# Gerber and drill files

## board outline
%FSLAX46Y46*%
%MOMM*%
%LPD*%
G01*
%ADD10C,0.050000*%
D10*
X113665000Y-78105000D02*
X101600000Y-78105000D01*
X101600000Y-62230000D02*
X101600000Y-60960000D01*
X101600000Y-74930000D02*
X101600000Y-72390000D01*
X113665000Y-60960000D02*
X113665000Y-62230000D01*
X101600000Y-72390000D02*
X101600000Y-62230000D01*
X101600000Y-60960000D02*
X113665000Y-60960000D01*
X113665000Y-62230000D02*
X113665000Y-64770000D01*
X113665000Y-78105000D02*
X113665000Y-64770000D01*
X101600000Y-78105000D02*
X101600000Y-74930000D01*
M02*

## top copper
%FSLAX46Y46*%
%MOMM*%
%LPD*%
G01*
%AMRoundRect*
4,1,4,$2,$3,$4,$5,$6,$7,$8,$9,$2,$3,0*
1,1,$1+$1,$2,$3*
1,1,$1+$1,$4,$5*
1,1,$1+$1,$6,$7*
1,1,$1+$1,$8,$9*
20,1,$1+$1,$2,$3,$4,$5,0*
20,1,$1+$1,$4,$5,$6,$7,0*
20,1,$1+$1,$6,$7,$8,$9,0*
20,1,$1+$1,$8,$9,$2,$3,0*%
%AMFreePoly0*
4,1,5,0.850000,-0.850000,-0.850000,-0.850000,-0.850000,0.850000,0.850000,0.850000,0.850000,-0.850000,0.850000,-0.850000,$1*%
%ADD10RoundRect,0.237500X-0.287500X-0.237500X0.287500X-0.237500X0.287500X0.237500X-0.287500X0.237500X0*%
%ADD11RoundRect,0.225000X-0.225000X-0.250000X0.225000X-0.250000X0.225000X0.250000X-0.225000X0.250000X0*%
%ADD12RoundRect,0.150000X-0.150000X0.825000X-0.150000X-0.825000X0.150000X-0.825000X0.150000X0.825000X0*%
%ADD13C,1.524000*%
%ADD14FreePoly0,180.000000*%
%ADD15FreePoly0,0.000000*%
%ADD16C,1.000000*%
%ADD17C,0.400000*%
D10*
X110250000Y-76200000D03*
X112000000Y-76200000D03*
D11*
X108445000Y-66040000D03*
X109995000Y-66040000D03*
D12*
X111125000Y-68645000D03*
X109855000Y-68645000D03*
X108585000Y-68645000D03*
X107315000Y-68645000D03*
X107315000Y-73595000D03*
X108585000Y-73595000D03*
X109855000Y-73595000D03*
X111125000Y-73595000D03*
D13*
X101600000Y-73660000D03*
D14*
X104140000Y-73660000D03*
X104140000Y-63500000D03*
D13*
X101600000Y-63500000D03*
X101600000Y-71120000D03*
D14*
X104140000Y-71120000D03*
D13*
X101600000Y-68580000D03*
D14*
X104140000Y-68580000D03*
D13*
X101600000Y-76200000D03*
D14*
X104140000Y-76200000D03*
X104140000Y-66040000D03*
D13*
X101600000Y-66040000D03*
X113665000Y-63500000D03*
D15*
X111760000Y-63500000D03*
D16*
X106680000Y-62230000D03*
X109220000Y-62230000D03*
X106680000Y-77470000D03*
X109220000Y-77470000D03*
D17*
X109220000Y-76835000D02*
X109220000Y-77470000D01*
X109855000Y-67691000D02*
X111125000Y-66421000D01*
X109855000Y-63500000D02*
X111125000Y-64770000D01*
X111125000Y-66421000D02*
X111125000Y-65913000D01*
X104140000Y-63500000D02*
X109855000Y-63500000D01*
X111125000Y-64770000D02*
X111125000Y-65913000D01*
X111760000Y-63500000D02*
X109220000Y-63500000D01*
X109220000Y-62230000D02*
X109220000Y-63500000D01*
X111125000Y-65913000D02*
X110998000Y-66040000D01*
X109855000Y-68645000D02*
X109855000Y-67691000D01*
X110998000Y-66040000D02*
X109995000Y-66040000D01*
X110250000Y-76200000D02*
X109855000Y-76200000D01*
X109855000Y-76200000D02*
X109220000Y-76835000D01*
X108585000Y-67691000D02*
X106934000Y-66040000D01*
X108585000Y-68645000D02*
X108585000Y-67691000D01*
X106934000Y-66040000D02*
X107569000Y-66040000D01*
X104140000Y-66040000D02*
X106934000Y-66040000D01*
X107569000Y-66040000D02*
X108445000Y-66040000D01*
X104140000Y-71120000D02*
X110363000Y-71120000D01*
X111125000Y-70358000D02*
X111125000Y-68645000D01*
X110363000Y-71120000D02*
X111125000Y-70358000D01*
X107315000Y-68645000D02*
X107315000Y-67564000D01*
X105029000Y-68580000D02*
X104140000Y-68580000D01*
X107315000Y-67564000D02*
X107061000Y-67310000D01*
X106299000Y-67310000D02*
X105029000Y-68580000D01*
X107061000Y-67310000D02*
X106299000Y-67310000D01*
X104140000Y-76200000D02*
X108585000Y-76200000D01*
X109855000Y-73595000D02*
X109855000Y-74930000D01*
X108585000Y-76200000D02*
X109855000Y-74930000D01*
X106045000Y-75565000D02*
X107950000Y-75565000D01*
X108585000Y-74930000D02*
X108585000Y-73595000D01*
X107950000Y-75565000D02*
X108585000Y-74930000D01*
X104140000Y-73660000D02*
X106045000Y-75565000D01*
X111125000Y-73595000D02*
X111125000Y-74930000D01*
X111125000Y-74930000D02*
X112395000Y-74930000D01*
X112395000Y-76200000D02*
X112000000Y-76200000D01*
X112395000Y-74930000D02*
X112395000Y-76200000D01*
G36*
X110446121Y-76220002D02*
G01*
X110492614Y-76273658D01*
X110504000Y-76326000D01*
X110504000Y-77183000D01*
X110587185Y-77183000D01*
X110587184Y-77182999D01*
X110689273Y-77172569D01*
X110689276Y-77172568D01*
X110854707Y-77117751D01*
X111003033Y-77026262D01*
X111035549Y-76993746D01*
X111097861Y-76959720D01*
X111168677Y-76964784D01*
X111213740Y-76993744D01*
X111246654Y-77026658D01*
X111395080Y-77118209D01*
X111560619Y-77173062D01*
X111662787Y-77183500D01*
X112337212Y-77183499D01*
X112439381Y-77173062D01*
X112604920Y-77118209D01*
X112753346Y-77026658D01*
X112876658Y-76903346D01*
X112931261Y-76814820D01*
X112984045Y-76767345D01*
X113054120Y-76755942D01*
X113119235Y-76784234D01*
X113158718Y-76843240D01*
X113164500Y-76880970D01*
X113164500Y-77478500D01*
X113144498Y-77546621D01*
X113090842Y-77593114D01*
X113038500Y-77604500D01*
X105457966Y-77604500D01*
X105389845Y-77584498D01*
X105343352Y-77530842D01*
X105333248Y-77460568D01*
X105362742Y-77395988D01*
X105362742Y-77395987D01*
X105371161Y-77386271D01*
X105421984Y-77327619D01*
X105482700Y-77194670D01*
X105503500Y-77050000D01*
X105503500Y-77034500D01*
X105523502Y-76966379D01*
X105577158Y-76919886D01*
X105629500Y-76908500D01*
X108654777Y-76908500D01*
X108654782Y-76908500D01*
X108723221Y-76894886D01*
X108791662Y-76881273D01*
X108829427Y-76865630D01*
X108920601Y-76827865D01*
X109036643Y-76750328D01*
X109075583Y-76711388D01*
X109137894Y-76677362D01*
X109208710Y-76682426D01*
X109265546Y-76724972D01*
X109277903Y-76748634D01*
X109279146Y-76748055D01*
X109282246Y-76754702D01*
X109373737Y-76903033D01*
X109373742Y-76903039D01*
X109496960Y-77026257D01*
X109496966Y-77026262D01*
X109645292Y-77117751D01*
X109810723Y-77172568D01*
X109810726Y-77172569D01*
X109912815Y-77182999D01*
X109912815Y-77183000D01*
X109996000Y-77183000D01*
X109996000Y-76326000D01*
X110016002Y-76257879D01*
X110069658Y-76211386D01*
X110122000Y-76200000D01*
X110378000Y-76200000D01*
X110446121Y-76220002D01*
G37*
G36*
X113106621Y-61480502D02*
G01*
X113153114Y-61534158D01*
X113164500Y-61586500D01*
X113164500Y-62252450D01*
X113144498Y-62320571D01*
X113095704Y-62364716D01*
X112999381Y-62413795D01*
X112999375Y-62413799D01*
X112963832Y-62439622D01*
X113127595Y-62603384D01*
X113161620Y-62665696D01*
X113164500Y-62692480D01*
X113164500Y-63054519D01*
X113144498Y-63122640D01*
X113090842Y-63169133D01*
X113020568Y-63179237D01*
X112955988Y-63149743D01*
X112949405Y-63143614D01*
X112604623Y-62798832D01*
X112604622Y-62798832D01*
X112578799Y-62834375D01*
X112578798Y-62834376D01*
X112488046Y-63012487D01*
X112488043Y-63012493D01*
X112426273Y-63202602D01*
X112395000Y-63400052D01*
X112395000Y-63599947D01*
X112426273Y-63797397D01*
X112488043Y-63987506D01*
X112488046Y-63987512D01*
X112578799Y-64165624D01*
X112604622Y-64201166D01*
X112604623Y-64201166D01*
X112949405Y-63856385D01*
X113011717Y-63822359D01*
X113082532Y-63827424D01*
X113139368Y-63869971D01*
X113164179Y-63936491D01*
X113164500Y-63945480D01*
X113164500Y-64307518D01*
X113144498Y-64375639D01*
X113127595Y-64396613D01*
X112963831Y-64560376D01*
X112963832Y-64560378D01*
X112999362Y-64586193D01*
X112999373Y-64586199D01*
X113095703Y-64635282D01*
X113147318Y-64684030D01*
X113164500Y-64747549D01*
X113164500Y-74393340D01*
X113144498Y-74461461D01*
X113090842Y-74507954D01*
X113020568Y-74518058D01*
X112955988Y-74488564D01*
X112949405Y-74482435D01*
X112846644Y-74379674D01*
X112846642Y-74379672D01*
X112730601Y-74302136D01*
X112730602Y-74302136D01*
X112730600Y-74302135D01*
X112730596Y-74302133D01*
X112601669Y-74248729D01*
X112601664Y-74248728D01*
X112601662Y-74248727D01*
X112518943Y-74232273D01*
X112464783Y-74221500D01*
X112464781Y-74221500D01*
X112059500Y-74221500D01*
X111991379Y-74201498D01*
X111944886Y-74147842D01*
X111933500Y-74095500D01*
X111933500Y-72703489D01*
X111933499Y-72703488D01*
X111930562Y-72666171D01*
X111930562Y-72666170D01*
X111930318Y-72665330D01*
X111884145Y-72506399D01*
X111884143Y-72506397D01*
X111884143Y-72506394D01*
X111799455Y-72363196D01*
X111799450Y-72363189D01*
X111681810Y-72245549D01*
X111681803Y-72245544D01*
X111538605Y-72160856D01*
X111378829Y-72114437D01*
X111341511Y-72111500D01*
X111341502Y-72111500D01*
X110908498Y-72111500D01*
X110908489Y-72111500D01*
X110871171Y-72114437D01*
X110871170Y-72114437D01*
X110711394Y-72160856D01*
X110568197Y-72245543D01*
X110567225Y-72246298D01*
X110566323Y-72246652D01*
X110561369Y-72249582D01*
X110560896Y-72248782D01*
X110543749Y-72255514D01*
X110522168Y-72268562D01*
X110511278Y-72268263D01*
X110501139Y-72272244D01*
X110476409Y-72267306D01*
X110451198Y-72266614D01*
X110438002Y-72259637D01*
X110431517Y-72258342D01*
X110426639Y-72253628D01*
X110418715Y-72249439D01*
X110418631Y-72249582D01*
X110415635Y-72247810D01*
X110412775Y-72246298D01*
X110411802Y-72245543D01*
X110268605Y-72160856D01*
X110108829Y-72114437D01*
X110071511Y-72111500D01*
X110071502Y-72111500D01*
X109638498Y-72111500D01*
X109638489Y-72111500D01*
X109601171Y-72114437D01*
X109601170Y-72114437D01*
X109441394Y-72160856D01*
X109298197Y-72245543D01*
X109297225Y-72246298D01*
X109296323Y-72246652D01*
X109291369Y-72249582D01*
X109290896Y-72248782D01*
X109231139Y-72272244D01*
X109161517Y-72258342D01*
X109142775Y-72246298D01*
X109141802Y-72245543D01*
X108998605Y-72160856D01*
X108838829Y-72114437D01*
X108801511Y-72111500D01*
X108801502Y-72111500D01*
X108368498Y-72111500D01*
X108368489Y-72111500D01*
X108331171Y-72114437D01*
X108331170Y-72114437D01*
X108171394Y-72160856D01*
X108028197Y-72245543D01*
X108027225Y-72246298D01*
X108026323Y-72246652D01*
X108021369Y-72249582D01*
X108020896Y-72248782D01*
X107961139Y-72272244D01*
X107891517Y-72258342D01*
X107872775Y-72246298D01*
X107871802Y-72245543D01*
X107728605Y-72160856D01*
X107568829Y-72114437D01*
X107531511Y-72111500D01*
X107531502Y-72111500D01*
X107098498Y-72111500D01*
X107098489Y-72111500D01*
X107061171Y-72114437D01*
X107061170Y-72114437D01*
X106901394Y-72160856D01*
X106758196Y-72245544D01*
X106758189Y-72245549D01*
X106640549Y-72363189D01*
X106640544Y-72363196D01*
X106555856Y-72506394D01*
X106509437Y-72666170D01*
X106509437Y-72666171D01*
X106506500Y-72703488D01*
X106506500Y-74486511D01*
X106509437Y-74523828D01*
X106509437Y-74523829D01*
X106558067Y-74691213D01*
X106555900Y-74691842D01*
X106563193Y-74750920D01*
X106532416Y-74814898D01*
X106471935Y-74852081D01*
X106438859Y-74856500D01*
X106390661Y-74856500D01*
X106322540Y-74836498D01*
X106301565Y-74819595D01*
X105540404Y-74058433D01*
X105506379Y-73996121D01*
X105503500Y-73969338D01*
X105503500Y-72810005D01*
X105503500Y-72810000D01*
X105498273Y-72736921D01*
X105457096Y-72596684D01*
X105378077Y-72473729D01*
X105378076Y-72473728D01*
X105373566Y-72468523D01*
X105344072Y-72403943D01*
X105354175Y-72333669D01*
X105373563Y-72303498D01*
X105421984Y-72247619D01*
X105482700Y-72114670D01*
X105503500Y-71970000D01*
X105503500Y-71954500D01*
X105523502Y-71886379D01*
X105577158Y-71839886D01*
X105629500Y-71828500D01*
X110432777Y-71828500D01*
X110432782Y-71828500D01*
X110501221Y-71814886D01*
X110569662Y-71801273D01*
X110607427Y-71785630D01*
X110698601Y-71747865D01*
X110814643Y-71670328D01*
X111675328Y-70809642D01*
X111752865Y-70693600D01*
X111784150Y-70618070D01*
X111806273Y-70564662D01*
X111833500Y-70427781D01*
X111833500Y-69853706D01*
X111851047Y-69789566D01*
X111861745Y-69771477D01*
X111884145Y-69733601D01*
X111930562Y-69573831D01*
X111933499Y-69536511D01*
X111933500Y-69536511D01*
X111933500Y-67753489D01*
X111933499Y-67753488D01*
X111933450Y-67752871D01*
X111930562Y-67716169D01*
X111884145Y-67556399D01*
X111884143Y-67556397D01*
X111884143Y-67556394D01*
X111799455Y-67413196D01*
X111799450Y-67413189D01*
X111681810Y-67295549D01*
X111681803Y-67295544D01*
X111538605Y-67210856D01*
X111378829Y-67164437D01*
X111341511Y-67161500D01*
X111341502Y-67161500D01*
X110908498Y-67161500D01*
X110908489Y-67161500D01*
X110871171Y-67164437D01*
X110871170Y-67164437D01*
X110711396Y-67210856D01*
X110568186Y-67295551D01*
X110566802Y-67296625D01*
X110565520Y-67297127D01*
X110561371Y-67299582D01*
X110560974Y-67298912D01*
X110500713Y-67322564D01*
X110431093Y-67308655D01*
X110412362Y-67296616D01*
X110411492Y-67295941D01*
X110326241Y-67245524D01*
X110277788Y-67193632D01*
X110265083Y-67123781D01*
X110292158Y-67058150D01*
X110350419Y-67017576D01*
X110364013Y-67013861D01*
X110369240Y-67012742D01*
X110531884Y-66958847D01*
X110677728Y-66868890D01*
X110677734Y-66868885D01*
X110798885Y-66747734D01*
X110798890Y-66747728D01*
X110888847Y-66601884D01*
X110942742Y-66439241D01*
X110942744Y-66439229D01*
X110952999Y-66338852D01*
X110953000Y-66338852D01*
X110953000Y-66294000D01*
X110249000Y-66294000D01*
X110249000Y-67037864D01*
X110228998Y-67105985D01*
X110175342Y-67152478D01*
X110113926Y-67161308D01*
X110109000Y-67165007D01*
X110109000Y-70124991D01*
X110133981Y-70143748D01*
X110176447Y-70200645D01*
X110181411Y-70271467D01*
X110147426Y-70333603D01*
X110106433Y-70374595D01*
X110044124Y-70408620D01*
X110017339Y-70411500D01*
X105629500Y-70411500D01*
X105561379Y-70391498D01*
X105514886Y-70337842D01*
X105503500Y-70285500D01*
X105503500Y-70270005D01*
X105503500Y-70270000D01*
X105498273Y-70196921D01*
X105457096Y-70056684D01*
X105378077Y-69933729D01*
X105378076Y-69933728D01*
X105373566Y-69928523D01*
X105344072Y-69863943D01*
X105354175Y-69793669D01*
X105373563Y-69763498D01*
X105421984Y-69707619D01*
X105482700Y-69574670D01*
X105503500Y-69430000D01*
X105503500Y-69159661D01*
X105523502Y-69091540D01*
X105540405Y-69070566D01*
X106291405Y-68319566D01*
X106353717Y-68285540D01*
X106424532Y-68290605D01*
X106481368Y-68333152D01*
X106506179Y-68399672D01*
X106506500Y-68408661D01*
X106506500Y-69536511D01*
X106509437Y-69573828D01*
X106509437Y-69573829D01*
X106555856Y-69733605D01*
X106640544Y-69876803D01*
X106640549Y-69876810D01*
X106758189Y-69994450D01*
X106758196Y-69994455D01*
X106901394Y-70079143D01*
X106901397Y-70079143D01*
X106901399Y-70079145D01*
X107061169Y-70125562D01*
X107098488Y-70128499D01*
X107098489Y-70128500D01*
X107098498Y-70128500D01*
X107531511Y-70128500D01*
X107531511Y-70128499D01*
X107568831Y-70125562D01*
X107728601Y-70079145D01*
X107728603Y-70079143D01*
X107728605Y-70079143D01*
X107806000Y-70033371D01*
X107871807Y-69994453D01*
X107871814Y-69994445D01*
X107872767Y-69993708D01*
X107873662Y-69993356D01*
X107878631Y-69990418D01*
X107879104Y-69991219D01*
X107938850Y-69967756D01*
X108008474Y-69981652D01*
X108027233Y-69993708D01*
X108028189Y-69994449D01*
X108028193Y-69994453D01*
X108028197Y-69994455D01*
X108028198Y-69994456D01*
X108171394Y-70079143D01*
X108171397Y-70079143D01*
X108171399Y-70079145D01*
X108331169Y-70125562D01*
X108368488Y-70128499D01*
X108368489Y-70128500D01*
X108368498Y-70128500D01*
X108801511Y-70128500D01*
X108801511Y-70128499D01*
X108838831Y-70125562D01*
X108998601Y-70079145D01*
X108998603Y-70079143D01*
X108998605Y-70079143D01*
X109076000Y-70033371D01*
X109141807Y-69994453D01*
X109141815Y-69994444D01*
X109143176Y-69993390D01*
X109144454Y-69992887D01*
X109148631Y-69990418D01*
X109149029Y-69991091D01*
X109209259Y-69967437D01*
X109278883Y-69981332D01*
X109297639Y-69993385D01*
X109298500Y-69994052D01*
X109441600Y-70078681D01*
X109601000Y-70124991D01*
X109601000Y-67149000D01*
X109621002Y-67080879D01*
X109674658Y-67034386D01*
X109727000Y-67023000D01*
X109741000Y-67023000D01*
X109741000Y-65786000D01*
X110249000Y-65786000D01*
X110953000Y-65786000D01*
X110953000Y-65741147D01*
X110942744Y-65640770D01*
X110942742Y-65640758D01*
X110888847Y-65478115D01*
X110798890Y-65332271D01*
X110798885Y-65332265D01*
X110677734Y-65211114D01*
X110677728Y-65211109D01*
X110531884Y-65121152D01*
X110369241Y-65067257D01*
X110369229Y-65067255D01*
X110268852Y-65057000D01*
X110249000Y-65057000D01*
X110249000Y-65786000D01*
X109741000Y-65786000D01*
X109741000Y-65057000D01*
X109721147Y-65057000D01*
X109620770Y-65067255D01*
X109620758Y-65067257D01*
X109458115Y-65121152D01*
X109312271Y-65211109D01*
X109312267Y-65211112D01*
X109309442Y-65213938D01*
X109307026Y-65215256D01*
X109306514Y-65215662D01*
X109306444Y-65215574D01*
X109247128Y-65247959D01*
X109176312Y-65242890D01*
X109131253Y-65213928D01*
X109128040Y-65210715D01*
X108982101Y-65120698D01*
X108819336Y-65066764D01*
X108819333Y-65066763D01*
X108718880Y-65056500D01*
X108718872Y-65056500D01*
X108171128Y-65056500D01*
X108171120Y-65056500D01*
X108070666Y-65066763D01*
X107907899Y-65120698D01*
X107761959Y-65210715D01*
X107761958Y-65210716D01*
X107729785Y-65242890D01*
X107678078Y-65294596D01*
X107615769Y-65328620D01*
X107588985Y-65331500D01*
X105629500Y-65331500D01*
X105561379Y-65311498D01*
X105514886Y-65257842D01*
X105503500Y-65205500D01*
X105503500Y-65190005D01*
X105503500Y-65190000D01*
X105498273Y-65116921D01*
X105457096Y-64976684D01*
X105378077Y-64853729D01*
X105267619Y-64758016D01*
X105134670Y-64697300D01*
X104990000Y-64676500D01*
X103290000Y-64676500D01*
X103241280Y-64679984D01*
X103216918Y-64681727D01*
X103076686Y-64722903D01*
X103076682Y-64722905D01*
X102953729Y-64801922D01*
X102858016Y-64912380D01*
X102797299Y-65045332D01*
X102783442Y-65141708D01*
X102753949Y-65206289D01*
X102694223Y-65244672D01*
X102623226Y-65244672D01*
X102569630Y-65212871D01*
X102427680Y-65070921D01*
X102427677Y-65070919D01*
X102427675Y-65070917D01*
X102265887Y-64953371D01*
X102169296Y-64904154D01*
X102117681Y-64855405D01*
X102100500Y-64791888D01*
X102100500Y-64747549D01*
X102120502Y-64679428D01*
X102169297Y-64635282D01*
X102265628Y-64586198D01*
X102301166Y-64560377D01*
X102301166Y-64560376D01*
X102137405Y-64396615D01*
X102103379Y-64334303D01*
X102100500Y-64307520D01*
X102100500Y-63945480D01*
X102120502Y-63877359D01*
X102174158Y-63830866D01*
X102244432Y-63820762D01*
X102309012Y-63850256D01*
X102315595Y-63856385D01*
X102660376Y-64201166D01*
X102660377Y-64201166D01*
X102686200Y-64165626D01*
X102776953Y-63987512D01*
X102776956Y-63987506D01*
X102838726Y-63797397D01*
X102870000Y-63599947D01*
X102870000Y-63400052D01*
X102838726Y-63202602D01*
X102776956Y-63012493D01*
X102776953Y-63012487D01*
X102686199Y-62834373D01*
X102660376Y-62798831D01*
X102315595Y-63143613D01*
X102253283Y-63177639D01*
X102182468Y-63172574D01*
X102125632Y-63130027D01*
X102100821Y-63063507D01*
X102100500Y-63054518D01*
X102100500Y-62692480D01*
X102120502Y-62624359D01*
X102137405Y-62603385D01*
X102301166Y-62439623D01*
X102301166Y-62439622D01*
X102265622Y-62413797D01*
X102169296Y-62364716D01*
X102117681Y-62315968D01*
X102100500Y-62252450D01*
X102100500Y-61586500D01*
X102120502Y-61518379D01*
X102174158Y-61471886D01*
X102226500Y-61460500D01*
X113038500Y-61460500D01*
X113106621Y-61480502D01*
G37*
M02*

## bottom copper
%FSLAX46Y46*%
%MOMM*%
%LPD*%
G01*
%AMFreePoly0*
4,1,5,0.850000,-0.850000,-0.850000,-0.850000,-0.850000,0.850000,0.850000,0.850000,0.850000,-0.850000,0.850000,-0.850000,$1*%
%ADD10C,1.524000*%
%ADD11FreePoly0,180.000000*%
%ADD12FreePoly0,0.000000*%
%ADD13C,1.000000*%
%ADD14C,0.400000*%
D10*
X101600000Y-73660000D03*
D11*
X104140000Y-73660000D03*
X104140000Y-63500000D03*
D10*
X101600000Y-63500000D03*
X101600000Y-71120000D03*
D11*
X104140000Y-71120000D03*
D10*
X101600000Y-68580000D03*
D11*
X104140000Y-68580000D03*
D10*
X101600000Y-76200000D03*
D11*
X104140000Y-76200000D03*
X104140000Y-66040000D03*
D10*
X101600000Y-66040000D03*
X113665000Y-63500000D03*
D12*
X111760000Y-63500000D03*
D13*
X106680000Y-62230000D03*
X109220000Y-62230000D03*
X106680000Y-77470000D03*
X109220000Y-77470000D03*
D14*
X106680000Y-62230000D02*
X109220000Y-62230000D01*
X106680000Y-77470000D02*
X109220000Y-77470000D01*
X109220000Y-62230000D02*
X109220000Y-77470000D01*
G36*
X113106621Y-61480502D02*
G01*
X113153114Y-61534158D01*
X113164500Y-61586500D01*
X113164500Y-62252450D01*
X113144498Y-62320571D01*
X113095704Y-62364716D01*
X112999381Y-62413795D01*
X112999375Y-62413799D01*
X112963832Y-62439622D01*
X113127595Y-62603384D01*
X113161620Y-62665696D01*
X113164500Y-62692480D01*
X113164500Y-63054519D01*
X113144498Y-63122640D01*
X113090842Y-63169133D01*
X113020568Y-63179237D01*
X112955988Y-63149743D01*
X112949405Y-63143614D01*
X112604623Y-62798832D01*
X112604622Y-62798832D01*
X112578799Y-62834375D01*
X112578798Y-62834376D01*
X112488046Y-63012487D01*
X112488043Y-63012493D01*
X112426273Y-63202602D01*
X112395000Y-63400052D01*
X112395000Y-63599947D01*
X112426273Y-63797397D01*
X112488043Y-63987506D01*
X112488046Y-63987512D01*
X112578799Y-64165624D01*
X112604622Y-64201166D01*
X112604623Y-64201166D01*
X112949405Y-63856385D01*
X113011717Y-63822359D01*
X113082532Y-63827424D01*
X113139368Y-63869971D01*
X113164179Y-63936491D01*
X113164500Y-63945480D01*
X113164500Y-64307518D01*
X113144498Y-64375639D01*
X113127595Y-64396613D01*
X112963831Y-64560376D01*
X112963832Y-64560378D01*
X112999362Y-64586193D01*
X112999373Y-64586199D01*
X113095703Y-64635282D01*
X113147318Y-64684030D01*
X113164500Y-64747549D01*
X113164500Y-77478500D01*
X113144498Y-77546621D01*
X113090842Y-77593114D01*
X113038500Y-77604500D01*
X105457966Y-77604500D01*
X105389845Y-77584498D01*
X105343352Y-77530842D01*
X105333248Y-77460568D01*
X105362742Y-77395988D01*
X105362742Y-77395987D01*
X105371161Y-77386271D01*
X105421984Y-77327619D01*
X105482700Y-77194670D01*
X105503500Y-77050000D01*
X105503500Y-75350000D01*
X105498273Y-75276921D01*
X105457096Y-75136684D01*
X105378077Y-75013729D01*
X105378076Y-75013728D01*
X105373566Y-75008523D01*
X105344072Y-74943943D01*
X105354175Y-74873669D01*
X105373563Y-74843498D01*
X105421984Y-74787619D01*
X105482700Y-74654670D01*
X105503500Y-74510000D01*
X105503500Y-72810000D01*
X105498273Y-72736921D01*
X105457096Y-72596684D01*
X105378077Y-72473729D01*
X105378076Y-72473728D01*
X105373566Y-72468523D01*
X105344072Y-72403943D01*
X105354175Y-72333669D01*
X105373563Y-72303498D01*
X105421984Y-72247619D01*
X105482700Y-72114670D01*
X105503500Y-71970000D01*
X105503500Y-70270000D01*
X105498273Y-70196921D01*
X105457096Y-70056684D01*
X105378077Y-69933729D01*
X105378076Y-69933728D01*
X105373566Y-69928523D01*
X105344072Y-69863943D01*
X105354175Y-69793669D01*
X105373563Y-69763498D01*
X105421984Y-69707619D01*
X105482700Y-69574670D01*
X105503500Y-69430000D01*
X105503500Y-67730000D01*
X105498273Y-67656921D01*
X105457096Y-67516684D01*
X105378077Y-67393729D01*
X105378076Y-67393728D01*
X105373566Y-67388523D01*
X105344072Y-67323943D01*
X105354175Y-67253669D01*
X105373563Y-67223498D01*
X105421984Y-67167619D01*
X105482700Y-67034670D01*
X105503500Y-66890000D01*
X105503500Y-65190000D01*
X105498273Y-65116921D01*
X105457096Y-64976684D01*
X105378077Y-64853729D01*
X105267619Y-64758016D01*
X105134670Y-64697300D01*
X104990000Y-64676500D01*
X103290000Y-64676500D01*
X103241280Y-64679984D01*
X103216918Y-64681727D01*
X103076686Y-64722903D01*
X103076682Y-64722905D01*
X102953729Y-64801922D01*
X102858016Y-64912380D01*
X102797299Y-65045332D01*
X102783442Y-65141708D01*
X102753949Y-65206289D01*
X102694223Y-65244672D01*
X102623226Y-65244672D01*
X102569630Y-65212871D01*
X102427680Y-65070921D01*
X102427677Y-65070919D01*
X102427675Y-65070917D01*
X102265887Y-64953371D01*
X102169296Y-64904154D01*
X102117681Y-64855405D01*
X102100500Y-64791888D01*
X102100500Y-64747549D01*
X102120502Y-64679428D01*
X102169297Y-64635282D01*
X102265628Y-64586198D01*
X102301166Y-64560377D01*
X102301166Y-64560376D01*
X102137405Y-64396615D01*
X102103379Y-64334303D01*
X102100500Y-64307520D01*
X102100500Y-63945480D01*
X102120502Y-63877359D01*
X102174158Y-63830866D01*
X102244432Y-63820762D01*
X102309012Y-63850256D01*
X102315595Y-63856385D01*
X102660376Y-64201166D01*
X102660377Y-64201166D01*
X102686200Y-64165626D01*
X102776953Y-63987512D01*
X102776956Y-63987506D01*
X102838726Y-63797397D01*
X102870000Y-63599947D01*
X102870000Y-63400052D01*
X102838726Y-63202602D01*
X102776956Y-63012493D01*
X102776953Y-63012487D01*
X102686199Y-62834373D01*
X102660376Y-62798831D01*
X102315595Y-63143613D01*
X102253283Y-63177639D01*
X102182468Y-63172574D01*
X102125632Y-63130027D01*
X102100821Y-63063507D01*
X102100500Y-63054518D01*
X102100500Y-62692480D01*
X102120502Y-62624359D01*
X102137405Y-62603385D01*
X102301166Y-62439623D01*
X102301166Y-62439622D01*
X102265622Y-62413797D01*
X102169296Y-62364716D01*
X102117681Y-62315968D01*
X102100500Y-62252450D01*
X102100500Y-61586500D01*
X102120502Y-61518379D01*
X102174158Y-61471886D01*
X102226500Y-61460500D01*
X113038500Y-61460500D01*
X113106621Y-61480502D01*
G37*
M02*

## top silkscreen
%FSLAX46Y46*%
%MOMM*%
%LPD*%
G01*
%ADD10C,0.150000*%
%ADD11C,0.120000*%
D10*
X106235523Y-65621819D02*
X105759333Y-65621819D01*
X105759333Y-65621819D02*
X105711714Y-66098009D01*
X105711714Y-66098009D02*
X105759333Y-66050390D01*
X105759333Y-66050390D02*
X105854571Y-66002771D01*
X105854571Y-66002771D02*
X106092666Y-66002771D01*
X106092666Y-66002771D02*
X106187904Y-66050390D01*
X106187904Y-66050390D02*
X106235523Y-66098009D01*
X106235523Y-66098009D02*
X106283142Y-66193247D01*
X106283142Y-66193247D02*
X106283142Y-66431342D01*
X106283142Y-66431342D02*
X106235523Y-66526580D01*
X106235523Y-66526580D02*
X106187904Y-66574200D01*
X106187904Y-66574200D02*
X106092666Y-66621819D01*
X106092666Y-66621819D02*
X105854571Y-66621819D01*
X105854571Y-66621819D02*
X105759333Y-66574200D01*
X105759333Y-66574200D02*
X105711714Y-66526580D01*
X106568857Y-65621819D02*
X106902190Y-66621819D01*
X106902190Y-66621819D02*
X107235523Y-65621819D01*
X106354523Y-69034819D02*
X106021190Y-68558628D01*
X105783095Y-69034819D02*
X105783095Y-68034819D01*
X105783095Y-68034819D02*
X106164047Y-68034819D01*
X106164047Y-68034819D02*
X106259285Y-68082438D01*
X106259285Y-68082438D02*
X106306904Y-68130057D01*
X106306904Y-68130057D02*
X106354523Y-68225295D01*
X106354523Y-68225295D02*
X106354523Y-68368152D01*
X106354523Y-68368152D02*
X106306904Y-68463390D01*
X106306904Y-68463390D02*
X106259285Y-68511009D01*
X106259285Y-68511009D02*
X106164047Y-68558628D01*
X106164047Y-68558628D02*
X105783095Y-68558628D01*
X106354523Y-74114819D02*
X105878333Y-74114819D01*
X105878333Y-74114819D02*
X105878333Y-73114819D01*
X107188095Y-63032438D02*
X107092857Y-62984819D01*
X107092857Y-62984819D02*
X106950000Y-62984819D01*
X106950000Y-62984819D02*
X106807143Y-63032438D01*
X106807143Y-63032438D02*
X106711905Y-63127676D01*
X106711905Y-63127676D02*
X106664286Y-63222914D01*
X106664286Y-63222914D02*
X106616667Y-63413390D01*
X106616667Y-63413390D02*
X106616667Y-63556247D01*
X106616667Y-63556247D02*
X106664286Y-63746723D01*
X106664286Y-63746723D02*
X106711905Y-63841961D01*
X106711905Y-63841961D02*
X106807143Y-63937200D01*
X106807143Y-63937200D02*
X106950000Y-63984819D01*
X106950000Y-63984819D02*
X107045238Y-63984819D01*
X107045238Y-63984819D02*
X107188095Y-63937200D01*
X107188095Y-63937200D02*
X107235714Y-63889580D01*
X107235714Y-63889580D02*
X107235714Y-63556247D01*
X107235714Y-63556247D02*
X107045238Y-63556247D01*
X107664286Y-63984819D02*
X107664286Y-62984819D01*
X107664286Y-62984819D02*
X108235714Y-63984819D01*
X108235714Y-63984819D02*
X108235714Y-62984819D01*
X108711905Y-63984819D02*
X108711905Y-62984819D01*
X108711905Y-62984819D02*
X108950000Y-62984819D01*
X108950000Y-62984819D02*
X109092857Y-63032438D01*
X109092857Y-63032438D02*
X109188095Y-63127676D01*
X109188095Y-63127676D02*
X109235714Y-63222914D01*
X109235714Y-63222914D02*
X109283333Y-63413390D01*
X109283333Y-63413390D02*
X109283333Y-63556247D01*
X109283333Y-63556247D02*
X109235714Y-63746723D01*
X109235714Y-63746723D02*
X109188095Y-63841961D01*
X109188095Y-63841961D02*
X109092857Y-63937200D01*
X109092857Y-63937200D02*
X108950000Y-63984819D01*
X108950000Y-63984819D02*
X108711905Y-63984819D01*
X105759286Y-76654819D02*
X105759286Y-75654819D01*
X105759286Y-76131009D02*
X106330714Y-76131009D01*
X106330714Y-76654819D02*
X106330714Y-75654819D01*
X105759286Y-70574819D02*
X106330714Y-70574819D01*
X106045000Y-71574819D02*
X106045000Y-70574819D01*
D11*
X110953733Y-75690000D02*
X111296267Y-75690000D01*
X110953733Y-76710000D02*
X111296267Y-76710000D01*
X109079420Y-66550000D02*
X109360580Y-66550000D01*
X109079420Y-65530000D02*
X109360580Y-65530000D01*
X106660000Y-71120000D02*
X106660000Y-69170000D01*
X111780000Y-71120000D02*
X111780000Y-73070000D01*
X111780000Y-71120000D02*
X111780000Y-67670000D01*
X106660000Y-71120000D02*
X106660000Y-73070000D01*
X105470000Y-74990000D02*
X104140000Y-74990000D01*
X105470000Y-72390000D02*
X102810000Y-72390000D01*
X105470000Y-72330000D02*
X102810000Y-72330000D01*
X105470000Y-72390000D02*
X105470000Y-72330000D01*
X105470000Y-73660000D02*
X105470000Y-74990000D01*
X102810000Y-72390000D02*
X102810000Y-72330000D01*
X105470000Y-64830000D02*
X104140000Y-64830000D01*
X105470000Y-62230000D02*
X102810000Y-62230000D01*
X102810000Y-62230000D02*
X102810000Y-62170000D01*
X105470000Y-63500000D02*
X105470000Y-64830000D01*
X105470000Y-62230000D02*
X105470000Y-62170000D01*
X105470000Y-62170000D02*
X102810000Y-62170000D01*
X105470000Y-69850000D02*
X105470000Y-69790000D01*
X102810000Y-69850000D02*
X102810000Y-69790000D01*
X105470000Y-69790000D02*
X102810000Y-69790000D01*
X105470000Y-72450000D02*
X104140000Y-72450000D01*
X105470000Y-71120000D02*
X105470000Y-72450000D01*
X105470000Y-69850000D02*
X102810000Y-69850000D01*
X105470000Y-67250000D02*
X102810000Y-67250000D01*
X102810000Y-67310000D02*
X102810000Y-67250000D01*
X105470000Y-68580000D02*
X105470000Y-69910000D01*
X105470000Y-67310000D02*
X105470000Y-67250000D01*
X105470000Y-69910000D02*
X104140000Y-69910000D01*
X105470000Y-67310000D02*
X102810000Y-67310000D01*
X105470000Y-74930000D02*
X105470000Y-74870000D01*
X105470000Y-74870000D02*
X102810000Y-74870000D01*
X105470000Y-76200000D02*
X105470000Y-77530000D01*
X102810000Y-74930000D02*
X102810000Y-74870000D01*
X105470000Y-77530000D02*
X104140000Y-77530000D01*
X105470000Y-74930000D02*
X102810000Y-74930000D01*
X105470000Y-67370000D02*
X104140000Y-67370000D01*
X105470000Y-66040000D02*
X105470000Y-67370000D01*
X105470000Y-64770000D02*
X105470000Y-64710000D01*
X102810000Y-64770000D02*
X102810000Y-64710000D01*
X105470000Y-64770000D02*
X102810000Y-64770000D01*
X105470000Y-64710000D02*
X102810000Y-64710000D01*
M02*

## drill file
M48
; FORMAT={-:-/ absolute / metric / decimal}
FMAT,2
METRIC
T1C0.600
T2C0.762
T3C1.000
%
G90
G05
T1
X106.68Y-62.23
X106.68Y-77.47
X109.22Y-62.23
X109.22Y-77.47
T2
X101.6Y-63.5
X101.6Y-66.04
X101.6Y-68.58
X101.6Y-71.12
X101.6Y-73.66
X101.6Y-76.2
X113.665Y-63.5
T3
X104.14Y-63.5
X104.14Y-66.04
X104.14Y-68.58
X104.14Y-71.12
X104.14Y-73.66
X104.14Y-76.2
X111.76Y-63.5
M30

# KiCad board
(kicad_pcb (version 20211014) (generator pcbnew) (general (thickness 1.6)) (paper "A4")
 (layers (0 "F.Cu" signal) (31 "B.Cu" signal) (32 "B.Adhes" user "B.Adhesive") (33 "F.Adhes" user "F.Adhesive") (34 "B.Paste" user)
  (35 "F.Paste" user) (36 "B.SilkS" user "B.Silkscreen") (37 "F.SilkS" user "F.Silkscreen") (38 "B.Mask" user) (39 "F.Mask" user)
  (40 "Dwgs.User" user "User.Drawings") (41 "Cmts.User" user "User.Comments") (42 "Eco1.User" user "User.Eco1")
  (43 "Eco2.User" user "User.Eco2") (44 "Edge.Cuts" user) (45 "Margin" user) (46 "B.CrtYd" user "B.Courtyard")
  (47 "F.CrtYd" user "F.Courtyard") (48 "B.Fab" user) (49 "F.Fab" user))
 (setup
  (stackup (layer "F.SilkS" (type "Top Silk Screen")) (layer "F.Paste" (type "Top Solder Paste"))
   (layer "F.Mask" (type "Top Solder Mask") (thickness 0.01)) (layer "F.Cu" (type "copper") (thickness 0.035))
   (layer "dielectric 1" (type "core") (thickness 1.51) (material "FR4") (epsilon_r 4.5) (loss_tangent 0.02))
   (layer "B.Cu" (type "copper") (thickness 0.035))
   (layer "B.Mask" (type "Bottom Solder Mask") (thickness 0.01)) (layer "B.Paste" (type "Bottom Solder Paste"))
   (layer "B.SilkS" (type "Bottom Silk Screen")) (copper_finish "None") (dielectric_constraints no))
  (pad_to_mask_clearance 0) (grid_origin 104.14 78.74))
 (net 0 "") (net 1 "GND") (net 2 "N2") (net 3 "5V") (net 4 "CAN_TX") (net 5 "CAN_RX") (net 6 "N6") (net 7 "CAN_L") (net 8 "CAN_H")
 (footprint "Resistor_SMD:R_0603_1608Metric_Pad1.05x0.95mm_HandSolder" (layer "F.Cu") (at 111.125 76.2)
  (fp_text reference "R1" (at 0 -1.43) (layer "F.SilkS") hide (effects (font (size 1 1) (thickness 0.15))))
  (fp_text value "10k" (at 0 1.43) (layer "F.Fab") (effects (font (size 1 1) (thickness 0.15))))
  (fp_line (start -0.171267 -0.51) (end 0.171267 -0.51) (layer "F.SilkS") (width 0.12))
  (fp_line (start -0.171267 0.51) (end 0.171267 0.51) (layer "F.SilkS") (width 0.12))
  (pad "1" smd roundrect locked (at -0.875 0) (size 1.05 0.95) (layers "F.Cu" "F.Paste" "F.Mask") (roundrect_rratio 0.25) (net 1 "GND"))
  (pad "2" smd roundrect locked (at 0.875 0) (size 1.05 0.95) (layers "F.Cu" "F.Paste" "F.Mask") (roundrect_rratio 0.25) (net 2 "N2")))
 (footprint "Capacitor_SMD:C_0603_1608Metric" (layer "F.Cu") (at 109.22 66.04)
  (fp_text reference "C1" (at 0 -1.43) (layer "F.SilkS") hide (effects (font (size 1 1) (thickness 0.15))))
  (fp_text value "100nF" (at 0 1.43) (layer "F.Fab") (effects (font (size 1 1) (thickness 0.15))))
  (fp_line (start -0.14058 0.51) (end 0.14058 0.51) (layer "F.SilkS") (width 0.12))
  (fp_line (start -0.14058 -0.51) (end 0.14058 -0.51) (layer "F.SilkS") (width 0.12))
  (pad "1" smd roundrect locked (at -0.775 0) (size 0.9 0.95) (layers "F.Cu" "F.Paste" "F.Mask") (roundrect_rratio 0.25) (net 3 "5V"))
  (pad "2" smd roundrect locked (at 0.775 0) (size 0.9 0.95) (layers "F.Cu" "F.Paste" "F.Mask") (roundrect_rratio 0.25) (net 1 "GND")))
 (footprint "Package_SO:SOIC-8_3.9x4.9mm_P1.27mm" (layer "F.Cu") (at 109.22 71.12 -90)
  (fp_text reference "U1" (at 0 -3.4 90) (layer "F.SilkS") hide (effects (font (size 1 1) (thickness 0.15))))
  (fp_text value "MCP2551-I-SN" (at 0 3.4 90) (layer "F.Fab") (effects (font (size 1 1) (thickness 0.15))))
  (fp_line (start 0 2.56) (end -1.95 2.56) (layer "F.SilkS") (width 0.12))
  (fp_line (start 0 -2.56) (end 1.95 -2.56) (layer "F.SilkS") (width 0.12))
  (fp_line (start 0 -2.56) (end -3.45 -2.56) (layer "F.SilkS") (width 0.12))
  (fp_line (start 0 2.56) (end 1.95 2.56) (layer "F.SilkS") (width 0.12))
  (pad "1" smd roundrect locked (at -2.475 -1.905 270) (size 1.95 0.6) (layers "F.Cu" "F.Paste" "F.Mask") (roundrect_rratio 0.25)
   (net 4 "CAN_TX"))
  (pad "2" smd roundrect locked (at -2.475 -0.635 270) (size 1.95 0.6) (layers "F.Cu" "F.Paste" "F.Mask") (roundrect_rratio 0.25)
   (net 1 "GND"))
  (pad "3" smd roundrect locked (at -2.475 0.635 270) (size 1.95 0.6) (layers "F.Cu" "F.Paste" "F.Mask") (roundrect_rratio 0.25)
   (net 3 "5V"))
  (pad "4" smd roundrect locked (at -2.475 1.905 270) (size 1.95 0.6) (layers "F.Cu" "F.Paste" "F.Mask") (roundrect_rratio 0.25)
   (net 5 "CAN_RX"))
  (pad "5" smd roundrect locked (at 2.475 1.905 270) (size 1.95 0.6) (layers "F.Cu" "F.Paste" "F.Mask") (roundrect_rratio 0.25) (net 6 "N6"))
  (pad "6" smd roundrect locked (at 2.475 0.635 270) (size 1.95 0.6) (layers "F.Cu" "F.Paste" "F.Mask") (roundrect_rratio 0.25)
   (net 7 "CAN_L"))
  (pad "7" smd roundrect locked (at 2.475 -0.635 270) (size 1.95 0.6) (layers "F.Cu" "F.Paste" "F.Mask") (roundrect_rratio 0.25)
   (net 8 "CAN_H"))
  (pad "8" smd roundrect locked (at 2.475 -1.905 270) (size 1.95 0.6) (layers "F.Cu" "F.Paste" "F.Mask") (roundrect_rratio 0.25)
   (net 2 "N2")))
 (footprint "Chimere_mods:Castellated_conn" (layer "F.Cu") (at 104.14 73.66 180)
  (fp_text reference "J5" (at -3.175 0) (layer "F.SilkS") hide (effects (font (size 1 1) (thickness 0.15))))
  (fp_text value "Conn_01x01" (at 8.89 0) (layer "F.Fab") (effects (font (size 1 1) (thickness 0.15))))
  (fp_line (start -1.33 -1.33) (end 0 -1.33) (layer "F.SilkS") (width 0.12))
  (fp_line (start -1.33 1.27) (end 1.33 1.27) (layer "F.SilkS") (width 0.12))
  (fp_line (start -1.33 1.33) (end 1.33 1.33) (layer "F.SilkS") (width 0.12))
  (fp_line (start -1.33 1.27) (end -1.33 1.33) (layer "F.SilkS") (width 0.12))
  (fp_line (start -1.33 0) (end -1.33 -1.33) (layer "F.SilkS") (width 0.12))
  (fp_line (start 1.33 1.27) (end 1.33 1.33) (layer "F.SilkS") (width 0.12))
  (pad "1" thru_hole circle locked (at 2.54 0 180) (size 1.524 1.524) (drill 0.762) (layers *.Cu *.Mask) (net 7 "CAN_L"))
  (pad "1" thru_hole custom locked (at 0 0 180) (size 1.7 1.7) (drill 1) (layers *.Cu *.Mask) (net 7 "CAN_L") (zone_connect 2)
   (options (clearance outline) (anchor rect)) (primitives)))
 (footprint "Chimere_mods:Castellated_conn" (layer "F.Cu") (at 104.14 63.5 180)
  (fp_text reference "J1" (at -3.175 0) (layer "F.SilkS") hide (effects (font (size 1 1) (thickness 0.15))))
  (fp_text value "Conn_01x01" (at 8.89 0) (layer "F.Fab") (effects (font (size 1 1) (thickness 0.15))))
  (fp_line (start -1.33 -1.33) (end 0 -1.33) (layer "F.SilkS") (width 0.12))
  (fp_line (start -1.33 1.27) (end 1.33 1.27) (layer "F.SilkS") (width 0.12))
  (fp_line (start 1.33 1.27) (end 1.33 1.33) (layer "F.SilkS") (width 0.12))
  (fp_line (start -1.33 0) (end -1.33 -1.33) (layer "F.SilkS") (width 0.12))
  (fp_line (start -1.33 1.27) (end -1.33 1.33) (layer "F.SilkS") (width 0.12))
  (fp_line (start -1.33 1.33) (end 1.33 1.33) (layer "F.SilkS") (width 0.12))
  (pad "1" thru_hole custom locked (at 0 0 180) (size 1.7 1.7) (drill 1) (layers *.Cu *.Mask) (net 1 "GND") (zone_connect 2)
   (options (clearance outline) (anchor rect)) (primitives))
  (pad "1" thru_hole circle locked (at 2.54 0 180) (size 1.524 1.524) (drill 0.762) (layers *.Cu *.Mask) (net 1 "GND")))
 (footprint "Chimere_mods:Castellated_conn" (layer "F.Cu") (at 104.14 71.12 180)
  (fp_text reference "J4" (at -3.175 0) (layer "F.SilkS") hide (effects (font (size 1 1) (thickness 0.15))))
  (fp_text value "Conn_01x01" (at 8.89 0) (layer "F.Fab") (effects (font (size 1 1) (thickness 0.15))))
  (fp_line (start -1.33 1.27) (end -1.33 1.33) (layer "F.SilkS") (width 0.12))
  (fp_line (start 1.33 1.27) (end 1.33 1.33) (layer "F.SilkS") (width 0.12))
  (fp_line (start -1.33 1.33) (end 1.33 1.33) (layer "F.SilkS") (width 0.12))
  (fp_line (start -1.33 -1.33) (end 0 -1.33) (layer "F.SilkS") (width 0.12))
  (fp_line (start -1.33 0) (end -1.33 -1.33) (layer "F.SilkS") (width 0.12))
  (fp_line (start -1.33 1.27) (end 1.33 1.27) (layer "F.SilkS") (width 0.12))
  (pad "1" thru_hole circle locked (at 2.54 0 180) (size 1.524 1.524) (drill 0.762) (layers *.Cu *.Mask) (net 4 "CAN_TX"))
  (pad "1" thru_hole custom locked (at 0 0 180) (size 1.7 1.7) (drill 1) (layers *.Cu *.Mask) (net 4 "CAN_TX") (zone_connect 2)
   (options (clearance outline) (anchor rect)) (primitives)))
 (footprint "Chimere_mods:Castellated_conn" (layer "F.Cu") (at 104.14 68.58 180)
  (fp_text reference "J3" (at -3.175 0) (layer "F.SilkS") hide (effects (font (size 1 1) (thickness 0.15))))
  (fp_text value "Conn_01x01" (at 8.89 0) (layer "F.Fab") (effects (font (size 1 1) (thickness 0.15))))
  (fp_line (start -1.33 1.33) (end 1.33 1.33) (layer "F.SilkS") (width 0.12))
  (fp_line (start 1.33 1.27) (end 1.33 1.33) (layer "F.SilkS") (width 0.12))
  (fp_line (start -1.33 0) (end -1.33 -1.33) (layer "F.SilkS") (width 0.12))
  (fp_line (start -1.33 1.27) (end -1.33 1.33) (layer "F.SilkS") (width 0.12))
  (fp_line (start -1.33 -1.33) (end 0 -1.33) (layer "F.SilkS") (width 0.12))
  (fp_line (start -1.33 1.27) (end 1.33 1.27) (layer "F.SilkS") (width 0.12))
  (pad "1" thru_hole circle locked (at 2.54 0 180) (size 1.524 1.524) (drill 0.762) (layers *.Cu *.Mask) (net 5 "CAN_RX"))
  (pad "1" thru_hole custom locked (at 0 0 180) (size 1.7 1.7) (drill 1) (layers *.Cu *.Mask) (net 5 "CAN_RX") (zone_connect 2)
   (options (clearance outline) (anchor rect)) (primitives)))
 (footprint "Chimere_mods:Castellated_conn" (layer "F.Cu") (at 104.14 76.2 180)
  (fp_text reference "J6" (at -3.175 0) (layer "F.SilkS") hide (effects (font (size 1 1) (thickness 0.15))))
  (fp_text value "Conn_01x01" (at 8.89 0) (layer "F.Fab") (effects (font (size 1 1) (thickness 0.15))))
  (fp_line (start -1.33 1.27) (end -1.33 1.33) (layer "F.SilkS") (width 0.12))
  (fp_line (start -1.33 1.33) (end 1.33 1.33) (layer "F.SilkS") (width 0.12))
  (fp_line (start -1.33 0) (end -1.33 -1.33) (layer "F.SilkS") (width 0.12))
  (fp_line (start 1.33 1.27) (end 1.33 1.33) (layer "F.SilkS") (width 0.12))
  (fp_line (start -1.33 -1.33) (end 0 -1.33) (layer "F.SilkS") (width 0.12))
  (fp_line (start -1.33 1.27) (end 1.33 1.27) (layer "F.SilkS") (width 0.12))
  (pad "1" thru_hole circle locked (at 2.54 0 180) (size 1.524 1.524) (drill 0.762) (layers *.Cu *.Mask) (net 8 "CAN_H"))
  (pad "1" thru_hole custom locked (at 0 0 180) (size 1.7 1.7) (drill 1) (layers *.Cu *.Mask) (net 8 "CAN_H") (zone_connect 2)
   (options (clearance outline) (anchor rect)) (primitives)))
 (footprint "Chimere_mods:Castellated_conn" (layer "F.Cu") (at 104.14 66.04 180)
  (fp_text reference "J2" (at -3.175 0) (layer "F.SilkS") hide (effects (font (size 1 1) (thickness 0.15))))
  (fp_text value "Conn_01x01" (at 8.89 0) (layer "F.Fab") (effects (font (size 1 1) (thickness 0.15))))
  (fp_line (start -1.33 -1.33) (end 0 -1.33) (layer "F.SilkS") (width 0.12))
  (fp_line (start -1.33 0) (end -1.33 -1.33) (layer "F.SilkS") (width 0.12))
  (fp_line (start -1.33 1.27) (end -1.33 1.33) (layer "F.SilkS") (width 0.12))
  (fp_line (start 1.33 1.27) (end 1.33 1.33) (layer "F.SilkS") (width 0.12))
  (fp_line (start -1.33 1.27) (end 1.33 1.27) (layer "F.SilkS") (width 0.12))
  (fp_line (start -1.33 1.33) (end 1.33 1.33) (layer "F.SilkS") (width 0.12))
  (pad "1" thru_hole custom locked (at 0 0 180) (size 1.7 1.7) (drill 1) (layers *.Cu *.Mask) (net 3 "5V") (zone_connect 2)
   (options (clearance outline) (anchor rect)) (primitives))
  (pad "1" thru_hole circle locked (at 2.54 0 180) (size 1.524 1.524) (drill 0.762) (layers *.Cu *.Mask) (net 3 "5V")))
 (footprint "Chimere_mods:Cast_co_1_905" (layer "B.Cu") (at 111.76 63.5)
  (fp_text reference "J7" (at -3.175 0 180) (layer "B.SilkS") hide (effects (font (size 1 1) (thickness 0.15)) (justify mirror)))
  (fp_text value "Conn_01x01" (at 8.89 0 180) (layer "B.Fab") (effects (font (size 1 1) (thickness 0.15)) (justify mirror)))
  (pad "1" thru_hole circle (at 1.905 0) (size 1.524 1.524) (drill 0.762) (layers *.Cu *.Mask) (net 1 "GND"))
  (pad "1" thru_hole custom (at 0 0) (size 1.7 1.7) (drill 1) (layers *.Cu *.Mask) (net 1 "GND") (zone_connect 2)
   (options (clearance outline) (anchor rect)) (primitives)))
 (gr_line (start 113.665 78.105) (end 101.6 78.105) (layer "Edge.Cuts") (width 0.05))
 (gr_line (start 101.6 62.23) (end 101.6 60.96) (layer "Edge.Cuts") (width 0.05))
 (gr_line (start 101.6 74.93) (end 101.6 72.39) (layer "Edge.Cuts") (width 0.05))
 (gr_line (start 113.665 60.96) (end 113.665 62.23) (layer "Edge.Cuts") (width 0.05))
 (gr_line (start 101.6 72.39) (end 101.6 62.23) (layer "Edge.Cuts") (width 0.05))
 (gr_line (start 101.6 60.96) (end 113.665 60.96) (layer "Edge.Cuts") (width 0.05))
 (gr_line (start 113.665 62.23) (end 113.665 64.77) (layer "Edge.Cuts") (width 0.05))
 (gr_line (start 113.665 78.105) (end 113.665 64.77) (layer "Edge.Cuts") (width 0.05))
 (gr_line (start 101.6 78.105) (end 101.6 74.93) (layer "Edge.Cuts") (width 0.05))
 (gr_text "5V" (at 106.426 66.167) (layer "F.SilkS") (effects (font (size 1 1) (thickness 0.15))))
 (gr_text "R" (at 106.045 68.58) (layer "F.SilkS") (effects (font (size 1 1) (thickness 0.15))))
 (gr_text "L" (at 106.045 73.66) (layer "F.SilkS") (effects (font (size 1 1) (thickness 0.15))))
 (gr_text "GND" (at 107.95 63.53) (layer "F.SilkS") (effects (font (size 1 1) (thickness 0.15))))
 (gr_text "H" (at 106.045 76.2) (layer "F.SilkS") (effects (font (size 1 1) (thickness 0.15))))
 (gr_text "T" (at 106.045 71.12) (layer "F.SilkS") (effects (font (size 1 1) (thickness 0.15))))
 (segment (start 109.22 76.835) (end 109.22 77.47) (width 0.4) (layer "F.Cu") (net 1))
 (segment (start 109.855 67.691) (end 111.125 66.421) (width 0.4) (layer "F.Cu") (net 1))
 (segment (start 109.855 63.5) (end 111.125 64.77) (width 0.4) (layer "F.Cu") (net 1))
 (segment (start 111.125 66.421) (end 111.125 65.913) (width 0.4) (layer "F.Cu") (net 1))
 (segment (start 104.14 63.5) (end 109.855 63.5) (width 0.4) (layer "F.Cu") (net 1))
 (segment (start 111.125 64.77) (end 111.125 65.913) (width 0.4) (layer "F.Cu") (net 1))
 (segment (start 111.76 63.5) (end 109.22 63.5) (width 0.4) (layer "F.Cu") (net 1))
 (segment (start 109.22 62.23) (end 109.22 63.5) (width 0.4) (layer "F.Cu") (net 1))
 (segment (start 111.125 65.913) (end 110.998 66.04) (width 0.4) (layer "F.Cu") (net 1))
 (segment (start 109.855 68.645) (end 109.855 67.691) (width 0.4) (layer "F.Cu") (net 1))
 (segment (start 110.998 66.04) (end 109.995 66.04) (width 0.4) (layer "F.Cu") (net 1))
 (segment (start 110.25 76.2) (end 109.855 76.2) (width 0.4) (layer "F.Cu") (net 1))
 (segment (start 109.855 76.2) (end 109.22 76.835) (width 0.4) (layer "F.Cu") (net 1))
 (via (at 106.68 62.23) (size 1) (drill 0.6) (layers "F.Cu" "B.Cu") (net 1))
 (via (at 109.22 62.23) (size 1) (drill 0.6) (layers "F.Cu" "B.Cu") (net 1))
 (via (at 106.68 77.47) (size 1) (drill 0.6) (layers "F.Cu" "B.Cu") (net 1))
 (via (at 109.22 77.47) (size 1) (drill 0.6) (layers "F.Cu" "B.Cu") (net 1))
 (segment (start 106.68 62.23) (end 109.22 62.23) (width 0.4) (layer "B.Cu") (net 1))
 (segment (start 106.68 77.47) (end 109.22 77.47) (width 0.4) (layer "B.Cu") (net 1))
 (segment (start 109.22 62.23) (end 109.22 77.47) (width 0.4) (layer "B.Cu") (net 1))
 (segment (start 108.585 67.691) (end 106.934 66.04) (width 0.4) (layer "F.Cu") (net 3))
 (segment (start 108.585 68.645) (end 108.585 67.691) (width 0.4) (layer "F.Cu") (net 3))
 (segment (start 106.934 66.04) (end 107.569 66.04) (width 0.4) (layer "F.Cu") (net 3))
 (segment (start 104.14 66.04) (end 106.934 66.04) (width 0.4) (layer "F.Cu") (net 3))
 (segment (start 107.569 66.04) (end 108.445 66.04) (width 0.4) (layer "F.Cu") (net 3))
 (segment (start 104.14 71.12) (end 110.363 71.12) (width 0.4) (layer "F.Cu") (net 4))
 (segment (start 111.125 70.358) (end 111.125 68.645) (width 0.4) (layer "F.Cu") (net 4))
 (segment (start 110.363 71.12) (end 111.125 70.358) (width 0.4) (layer "F.Cu") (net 4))
 (segment (start 107.315 68.645) (end 107.315 67.564) (width 0.4) (layer "F.Cu") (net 5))
 (segment (start 105.029 68.58) (end 104.14 68.58) (width 0.4) (layer "F.Cu") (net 5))
 (segment (start 107.315 67.564) (end 107.061 67.31) (width 0.4) (layer "F.Cu") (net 5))
 (segment (start 106.299 67.31) (end 105.029 68.58) (width 0.4) (layer "F.Cu") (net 5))
 (segment (start 107.061 67.31) (end 106.299 67.31) (width 0.4) (layer "F.Cu") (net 5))
 (segment (start 104.14 76.2) (end 108.585 76.2) (width 0.4) (layer "F.Cu") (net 8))
 (segment (start 109.855 73.595) (end 109.855 74.93) (width 0.4) (layer "F.Cu") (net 8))
 (segment (start 108.585 76.2) (end 109.855 74.93) (width 0.4) (layer "F.Cu") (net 8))
 (segment (start 106.045 75.565) (end 107.95 75.565) (width 0.4) (layer "F.Cu") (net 7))
 (segment (start 108.585 74.93) (end 108.585 73.595) (width 0.4) (layer "F.Cu") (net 7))
 (segment (start 107.95 75.565) (end 108.585 74.93) (width 0.4) (layer "F.Cu") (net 7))
 (segment (start 104.14 73.66) (end 106.045 75.565) (width 0.4) (layer "F.Cu") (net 7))
 (segment (start 111.125 73.595) (end 111.125 74.93) (width 0.4) (layer "F.Cu") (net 2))
 (segment (start 111.125 74.93) (end 112.395 74.93) (width 0.4) (layer "F.Cu") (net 2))
 (segment (start 112.395 76.2) (end 112 76.2) (width 0.4) (layer "F.Cu") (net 2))
 (segment (start 112.395 74.93) (end 112.395 76.2) (width 0.4) (layer "F.Cu") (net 2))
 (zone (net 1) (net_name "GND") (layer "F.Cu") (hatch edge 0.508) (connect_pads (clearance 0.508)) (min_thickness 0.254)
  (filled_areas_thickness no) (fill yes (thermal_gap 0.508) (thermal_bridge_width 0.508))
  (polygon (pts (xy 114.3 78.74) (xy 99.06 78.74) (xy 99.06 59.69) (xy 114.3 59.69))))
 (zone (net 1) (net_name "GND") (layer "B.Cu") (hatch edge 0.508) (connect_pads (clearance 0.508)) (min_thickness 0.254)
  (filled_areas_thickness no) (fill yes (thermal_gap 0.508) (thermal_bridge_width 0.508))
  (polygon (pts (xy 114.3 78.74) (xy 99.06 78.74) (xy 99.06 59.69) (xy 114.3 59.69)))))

